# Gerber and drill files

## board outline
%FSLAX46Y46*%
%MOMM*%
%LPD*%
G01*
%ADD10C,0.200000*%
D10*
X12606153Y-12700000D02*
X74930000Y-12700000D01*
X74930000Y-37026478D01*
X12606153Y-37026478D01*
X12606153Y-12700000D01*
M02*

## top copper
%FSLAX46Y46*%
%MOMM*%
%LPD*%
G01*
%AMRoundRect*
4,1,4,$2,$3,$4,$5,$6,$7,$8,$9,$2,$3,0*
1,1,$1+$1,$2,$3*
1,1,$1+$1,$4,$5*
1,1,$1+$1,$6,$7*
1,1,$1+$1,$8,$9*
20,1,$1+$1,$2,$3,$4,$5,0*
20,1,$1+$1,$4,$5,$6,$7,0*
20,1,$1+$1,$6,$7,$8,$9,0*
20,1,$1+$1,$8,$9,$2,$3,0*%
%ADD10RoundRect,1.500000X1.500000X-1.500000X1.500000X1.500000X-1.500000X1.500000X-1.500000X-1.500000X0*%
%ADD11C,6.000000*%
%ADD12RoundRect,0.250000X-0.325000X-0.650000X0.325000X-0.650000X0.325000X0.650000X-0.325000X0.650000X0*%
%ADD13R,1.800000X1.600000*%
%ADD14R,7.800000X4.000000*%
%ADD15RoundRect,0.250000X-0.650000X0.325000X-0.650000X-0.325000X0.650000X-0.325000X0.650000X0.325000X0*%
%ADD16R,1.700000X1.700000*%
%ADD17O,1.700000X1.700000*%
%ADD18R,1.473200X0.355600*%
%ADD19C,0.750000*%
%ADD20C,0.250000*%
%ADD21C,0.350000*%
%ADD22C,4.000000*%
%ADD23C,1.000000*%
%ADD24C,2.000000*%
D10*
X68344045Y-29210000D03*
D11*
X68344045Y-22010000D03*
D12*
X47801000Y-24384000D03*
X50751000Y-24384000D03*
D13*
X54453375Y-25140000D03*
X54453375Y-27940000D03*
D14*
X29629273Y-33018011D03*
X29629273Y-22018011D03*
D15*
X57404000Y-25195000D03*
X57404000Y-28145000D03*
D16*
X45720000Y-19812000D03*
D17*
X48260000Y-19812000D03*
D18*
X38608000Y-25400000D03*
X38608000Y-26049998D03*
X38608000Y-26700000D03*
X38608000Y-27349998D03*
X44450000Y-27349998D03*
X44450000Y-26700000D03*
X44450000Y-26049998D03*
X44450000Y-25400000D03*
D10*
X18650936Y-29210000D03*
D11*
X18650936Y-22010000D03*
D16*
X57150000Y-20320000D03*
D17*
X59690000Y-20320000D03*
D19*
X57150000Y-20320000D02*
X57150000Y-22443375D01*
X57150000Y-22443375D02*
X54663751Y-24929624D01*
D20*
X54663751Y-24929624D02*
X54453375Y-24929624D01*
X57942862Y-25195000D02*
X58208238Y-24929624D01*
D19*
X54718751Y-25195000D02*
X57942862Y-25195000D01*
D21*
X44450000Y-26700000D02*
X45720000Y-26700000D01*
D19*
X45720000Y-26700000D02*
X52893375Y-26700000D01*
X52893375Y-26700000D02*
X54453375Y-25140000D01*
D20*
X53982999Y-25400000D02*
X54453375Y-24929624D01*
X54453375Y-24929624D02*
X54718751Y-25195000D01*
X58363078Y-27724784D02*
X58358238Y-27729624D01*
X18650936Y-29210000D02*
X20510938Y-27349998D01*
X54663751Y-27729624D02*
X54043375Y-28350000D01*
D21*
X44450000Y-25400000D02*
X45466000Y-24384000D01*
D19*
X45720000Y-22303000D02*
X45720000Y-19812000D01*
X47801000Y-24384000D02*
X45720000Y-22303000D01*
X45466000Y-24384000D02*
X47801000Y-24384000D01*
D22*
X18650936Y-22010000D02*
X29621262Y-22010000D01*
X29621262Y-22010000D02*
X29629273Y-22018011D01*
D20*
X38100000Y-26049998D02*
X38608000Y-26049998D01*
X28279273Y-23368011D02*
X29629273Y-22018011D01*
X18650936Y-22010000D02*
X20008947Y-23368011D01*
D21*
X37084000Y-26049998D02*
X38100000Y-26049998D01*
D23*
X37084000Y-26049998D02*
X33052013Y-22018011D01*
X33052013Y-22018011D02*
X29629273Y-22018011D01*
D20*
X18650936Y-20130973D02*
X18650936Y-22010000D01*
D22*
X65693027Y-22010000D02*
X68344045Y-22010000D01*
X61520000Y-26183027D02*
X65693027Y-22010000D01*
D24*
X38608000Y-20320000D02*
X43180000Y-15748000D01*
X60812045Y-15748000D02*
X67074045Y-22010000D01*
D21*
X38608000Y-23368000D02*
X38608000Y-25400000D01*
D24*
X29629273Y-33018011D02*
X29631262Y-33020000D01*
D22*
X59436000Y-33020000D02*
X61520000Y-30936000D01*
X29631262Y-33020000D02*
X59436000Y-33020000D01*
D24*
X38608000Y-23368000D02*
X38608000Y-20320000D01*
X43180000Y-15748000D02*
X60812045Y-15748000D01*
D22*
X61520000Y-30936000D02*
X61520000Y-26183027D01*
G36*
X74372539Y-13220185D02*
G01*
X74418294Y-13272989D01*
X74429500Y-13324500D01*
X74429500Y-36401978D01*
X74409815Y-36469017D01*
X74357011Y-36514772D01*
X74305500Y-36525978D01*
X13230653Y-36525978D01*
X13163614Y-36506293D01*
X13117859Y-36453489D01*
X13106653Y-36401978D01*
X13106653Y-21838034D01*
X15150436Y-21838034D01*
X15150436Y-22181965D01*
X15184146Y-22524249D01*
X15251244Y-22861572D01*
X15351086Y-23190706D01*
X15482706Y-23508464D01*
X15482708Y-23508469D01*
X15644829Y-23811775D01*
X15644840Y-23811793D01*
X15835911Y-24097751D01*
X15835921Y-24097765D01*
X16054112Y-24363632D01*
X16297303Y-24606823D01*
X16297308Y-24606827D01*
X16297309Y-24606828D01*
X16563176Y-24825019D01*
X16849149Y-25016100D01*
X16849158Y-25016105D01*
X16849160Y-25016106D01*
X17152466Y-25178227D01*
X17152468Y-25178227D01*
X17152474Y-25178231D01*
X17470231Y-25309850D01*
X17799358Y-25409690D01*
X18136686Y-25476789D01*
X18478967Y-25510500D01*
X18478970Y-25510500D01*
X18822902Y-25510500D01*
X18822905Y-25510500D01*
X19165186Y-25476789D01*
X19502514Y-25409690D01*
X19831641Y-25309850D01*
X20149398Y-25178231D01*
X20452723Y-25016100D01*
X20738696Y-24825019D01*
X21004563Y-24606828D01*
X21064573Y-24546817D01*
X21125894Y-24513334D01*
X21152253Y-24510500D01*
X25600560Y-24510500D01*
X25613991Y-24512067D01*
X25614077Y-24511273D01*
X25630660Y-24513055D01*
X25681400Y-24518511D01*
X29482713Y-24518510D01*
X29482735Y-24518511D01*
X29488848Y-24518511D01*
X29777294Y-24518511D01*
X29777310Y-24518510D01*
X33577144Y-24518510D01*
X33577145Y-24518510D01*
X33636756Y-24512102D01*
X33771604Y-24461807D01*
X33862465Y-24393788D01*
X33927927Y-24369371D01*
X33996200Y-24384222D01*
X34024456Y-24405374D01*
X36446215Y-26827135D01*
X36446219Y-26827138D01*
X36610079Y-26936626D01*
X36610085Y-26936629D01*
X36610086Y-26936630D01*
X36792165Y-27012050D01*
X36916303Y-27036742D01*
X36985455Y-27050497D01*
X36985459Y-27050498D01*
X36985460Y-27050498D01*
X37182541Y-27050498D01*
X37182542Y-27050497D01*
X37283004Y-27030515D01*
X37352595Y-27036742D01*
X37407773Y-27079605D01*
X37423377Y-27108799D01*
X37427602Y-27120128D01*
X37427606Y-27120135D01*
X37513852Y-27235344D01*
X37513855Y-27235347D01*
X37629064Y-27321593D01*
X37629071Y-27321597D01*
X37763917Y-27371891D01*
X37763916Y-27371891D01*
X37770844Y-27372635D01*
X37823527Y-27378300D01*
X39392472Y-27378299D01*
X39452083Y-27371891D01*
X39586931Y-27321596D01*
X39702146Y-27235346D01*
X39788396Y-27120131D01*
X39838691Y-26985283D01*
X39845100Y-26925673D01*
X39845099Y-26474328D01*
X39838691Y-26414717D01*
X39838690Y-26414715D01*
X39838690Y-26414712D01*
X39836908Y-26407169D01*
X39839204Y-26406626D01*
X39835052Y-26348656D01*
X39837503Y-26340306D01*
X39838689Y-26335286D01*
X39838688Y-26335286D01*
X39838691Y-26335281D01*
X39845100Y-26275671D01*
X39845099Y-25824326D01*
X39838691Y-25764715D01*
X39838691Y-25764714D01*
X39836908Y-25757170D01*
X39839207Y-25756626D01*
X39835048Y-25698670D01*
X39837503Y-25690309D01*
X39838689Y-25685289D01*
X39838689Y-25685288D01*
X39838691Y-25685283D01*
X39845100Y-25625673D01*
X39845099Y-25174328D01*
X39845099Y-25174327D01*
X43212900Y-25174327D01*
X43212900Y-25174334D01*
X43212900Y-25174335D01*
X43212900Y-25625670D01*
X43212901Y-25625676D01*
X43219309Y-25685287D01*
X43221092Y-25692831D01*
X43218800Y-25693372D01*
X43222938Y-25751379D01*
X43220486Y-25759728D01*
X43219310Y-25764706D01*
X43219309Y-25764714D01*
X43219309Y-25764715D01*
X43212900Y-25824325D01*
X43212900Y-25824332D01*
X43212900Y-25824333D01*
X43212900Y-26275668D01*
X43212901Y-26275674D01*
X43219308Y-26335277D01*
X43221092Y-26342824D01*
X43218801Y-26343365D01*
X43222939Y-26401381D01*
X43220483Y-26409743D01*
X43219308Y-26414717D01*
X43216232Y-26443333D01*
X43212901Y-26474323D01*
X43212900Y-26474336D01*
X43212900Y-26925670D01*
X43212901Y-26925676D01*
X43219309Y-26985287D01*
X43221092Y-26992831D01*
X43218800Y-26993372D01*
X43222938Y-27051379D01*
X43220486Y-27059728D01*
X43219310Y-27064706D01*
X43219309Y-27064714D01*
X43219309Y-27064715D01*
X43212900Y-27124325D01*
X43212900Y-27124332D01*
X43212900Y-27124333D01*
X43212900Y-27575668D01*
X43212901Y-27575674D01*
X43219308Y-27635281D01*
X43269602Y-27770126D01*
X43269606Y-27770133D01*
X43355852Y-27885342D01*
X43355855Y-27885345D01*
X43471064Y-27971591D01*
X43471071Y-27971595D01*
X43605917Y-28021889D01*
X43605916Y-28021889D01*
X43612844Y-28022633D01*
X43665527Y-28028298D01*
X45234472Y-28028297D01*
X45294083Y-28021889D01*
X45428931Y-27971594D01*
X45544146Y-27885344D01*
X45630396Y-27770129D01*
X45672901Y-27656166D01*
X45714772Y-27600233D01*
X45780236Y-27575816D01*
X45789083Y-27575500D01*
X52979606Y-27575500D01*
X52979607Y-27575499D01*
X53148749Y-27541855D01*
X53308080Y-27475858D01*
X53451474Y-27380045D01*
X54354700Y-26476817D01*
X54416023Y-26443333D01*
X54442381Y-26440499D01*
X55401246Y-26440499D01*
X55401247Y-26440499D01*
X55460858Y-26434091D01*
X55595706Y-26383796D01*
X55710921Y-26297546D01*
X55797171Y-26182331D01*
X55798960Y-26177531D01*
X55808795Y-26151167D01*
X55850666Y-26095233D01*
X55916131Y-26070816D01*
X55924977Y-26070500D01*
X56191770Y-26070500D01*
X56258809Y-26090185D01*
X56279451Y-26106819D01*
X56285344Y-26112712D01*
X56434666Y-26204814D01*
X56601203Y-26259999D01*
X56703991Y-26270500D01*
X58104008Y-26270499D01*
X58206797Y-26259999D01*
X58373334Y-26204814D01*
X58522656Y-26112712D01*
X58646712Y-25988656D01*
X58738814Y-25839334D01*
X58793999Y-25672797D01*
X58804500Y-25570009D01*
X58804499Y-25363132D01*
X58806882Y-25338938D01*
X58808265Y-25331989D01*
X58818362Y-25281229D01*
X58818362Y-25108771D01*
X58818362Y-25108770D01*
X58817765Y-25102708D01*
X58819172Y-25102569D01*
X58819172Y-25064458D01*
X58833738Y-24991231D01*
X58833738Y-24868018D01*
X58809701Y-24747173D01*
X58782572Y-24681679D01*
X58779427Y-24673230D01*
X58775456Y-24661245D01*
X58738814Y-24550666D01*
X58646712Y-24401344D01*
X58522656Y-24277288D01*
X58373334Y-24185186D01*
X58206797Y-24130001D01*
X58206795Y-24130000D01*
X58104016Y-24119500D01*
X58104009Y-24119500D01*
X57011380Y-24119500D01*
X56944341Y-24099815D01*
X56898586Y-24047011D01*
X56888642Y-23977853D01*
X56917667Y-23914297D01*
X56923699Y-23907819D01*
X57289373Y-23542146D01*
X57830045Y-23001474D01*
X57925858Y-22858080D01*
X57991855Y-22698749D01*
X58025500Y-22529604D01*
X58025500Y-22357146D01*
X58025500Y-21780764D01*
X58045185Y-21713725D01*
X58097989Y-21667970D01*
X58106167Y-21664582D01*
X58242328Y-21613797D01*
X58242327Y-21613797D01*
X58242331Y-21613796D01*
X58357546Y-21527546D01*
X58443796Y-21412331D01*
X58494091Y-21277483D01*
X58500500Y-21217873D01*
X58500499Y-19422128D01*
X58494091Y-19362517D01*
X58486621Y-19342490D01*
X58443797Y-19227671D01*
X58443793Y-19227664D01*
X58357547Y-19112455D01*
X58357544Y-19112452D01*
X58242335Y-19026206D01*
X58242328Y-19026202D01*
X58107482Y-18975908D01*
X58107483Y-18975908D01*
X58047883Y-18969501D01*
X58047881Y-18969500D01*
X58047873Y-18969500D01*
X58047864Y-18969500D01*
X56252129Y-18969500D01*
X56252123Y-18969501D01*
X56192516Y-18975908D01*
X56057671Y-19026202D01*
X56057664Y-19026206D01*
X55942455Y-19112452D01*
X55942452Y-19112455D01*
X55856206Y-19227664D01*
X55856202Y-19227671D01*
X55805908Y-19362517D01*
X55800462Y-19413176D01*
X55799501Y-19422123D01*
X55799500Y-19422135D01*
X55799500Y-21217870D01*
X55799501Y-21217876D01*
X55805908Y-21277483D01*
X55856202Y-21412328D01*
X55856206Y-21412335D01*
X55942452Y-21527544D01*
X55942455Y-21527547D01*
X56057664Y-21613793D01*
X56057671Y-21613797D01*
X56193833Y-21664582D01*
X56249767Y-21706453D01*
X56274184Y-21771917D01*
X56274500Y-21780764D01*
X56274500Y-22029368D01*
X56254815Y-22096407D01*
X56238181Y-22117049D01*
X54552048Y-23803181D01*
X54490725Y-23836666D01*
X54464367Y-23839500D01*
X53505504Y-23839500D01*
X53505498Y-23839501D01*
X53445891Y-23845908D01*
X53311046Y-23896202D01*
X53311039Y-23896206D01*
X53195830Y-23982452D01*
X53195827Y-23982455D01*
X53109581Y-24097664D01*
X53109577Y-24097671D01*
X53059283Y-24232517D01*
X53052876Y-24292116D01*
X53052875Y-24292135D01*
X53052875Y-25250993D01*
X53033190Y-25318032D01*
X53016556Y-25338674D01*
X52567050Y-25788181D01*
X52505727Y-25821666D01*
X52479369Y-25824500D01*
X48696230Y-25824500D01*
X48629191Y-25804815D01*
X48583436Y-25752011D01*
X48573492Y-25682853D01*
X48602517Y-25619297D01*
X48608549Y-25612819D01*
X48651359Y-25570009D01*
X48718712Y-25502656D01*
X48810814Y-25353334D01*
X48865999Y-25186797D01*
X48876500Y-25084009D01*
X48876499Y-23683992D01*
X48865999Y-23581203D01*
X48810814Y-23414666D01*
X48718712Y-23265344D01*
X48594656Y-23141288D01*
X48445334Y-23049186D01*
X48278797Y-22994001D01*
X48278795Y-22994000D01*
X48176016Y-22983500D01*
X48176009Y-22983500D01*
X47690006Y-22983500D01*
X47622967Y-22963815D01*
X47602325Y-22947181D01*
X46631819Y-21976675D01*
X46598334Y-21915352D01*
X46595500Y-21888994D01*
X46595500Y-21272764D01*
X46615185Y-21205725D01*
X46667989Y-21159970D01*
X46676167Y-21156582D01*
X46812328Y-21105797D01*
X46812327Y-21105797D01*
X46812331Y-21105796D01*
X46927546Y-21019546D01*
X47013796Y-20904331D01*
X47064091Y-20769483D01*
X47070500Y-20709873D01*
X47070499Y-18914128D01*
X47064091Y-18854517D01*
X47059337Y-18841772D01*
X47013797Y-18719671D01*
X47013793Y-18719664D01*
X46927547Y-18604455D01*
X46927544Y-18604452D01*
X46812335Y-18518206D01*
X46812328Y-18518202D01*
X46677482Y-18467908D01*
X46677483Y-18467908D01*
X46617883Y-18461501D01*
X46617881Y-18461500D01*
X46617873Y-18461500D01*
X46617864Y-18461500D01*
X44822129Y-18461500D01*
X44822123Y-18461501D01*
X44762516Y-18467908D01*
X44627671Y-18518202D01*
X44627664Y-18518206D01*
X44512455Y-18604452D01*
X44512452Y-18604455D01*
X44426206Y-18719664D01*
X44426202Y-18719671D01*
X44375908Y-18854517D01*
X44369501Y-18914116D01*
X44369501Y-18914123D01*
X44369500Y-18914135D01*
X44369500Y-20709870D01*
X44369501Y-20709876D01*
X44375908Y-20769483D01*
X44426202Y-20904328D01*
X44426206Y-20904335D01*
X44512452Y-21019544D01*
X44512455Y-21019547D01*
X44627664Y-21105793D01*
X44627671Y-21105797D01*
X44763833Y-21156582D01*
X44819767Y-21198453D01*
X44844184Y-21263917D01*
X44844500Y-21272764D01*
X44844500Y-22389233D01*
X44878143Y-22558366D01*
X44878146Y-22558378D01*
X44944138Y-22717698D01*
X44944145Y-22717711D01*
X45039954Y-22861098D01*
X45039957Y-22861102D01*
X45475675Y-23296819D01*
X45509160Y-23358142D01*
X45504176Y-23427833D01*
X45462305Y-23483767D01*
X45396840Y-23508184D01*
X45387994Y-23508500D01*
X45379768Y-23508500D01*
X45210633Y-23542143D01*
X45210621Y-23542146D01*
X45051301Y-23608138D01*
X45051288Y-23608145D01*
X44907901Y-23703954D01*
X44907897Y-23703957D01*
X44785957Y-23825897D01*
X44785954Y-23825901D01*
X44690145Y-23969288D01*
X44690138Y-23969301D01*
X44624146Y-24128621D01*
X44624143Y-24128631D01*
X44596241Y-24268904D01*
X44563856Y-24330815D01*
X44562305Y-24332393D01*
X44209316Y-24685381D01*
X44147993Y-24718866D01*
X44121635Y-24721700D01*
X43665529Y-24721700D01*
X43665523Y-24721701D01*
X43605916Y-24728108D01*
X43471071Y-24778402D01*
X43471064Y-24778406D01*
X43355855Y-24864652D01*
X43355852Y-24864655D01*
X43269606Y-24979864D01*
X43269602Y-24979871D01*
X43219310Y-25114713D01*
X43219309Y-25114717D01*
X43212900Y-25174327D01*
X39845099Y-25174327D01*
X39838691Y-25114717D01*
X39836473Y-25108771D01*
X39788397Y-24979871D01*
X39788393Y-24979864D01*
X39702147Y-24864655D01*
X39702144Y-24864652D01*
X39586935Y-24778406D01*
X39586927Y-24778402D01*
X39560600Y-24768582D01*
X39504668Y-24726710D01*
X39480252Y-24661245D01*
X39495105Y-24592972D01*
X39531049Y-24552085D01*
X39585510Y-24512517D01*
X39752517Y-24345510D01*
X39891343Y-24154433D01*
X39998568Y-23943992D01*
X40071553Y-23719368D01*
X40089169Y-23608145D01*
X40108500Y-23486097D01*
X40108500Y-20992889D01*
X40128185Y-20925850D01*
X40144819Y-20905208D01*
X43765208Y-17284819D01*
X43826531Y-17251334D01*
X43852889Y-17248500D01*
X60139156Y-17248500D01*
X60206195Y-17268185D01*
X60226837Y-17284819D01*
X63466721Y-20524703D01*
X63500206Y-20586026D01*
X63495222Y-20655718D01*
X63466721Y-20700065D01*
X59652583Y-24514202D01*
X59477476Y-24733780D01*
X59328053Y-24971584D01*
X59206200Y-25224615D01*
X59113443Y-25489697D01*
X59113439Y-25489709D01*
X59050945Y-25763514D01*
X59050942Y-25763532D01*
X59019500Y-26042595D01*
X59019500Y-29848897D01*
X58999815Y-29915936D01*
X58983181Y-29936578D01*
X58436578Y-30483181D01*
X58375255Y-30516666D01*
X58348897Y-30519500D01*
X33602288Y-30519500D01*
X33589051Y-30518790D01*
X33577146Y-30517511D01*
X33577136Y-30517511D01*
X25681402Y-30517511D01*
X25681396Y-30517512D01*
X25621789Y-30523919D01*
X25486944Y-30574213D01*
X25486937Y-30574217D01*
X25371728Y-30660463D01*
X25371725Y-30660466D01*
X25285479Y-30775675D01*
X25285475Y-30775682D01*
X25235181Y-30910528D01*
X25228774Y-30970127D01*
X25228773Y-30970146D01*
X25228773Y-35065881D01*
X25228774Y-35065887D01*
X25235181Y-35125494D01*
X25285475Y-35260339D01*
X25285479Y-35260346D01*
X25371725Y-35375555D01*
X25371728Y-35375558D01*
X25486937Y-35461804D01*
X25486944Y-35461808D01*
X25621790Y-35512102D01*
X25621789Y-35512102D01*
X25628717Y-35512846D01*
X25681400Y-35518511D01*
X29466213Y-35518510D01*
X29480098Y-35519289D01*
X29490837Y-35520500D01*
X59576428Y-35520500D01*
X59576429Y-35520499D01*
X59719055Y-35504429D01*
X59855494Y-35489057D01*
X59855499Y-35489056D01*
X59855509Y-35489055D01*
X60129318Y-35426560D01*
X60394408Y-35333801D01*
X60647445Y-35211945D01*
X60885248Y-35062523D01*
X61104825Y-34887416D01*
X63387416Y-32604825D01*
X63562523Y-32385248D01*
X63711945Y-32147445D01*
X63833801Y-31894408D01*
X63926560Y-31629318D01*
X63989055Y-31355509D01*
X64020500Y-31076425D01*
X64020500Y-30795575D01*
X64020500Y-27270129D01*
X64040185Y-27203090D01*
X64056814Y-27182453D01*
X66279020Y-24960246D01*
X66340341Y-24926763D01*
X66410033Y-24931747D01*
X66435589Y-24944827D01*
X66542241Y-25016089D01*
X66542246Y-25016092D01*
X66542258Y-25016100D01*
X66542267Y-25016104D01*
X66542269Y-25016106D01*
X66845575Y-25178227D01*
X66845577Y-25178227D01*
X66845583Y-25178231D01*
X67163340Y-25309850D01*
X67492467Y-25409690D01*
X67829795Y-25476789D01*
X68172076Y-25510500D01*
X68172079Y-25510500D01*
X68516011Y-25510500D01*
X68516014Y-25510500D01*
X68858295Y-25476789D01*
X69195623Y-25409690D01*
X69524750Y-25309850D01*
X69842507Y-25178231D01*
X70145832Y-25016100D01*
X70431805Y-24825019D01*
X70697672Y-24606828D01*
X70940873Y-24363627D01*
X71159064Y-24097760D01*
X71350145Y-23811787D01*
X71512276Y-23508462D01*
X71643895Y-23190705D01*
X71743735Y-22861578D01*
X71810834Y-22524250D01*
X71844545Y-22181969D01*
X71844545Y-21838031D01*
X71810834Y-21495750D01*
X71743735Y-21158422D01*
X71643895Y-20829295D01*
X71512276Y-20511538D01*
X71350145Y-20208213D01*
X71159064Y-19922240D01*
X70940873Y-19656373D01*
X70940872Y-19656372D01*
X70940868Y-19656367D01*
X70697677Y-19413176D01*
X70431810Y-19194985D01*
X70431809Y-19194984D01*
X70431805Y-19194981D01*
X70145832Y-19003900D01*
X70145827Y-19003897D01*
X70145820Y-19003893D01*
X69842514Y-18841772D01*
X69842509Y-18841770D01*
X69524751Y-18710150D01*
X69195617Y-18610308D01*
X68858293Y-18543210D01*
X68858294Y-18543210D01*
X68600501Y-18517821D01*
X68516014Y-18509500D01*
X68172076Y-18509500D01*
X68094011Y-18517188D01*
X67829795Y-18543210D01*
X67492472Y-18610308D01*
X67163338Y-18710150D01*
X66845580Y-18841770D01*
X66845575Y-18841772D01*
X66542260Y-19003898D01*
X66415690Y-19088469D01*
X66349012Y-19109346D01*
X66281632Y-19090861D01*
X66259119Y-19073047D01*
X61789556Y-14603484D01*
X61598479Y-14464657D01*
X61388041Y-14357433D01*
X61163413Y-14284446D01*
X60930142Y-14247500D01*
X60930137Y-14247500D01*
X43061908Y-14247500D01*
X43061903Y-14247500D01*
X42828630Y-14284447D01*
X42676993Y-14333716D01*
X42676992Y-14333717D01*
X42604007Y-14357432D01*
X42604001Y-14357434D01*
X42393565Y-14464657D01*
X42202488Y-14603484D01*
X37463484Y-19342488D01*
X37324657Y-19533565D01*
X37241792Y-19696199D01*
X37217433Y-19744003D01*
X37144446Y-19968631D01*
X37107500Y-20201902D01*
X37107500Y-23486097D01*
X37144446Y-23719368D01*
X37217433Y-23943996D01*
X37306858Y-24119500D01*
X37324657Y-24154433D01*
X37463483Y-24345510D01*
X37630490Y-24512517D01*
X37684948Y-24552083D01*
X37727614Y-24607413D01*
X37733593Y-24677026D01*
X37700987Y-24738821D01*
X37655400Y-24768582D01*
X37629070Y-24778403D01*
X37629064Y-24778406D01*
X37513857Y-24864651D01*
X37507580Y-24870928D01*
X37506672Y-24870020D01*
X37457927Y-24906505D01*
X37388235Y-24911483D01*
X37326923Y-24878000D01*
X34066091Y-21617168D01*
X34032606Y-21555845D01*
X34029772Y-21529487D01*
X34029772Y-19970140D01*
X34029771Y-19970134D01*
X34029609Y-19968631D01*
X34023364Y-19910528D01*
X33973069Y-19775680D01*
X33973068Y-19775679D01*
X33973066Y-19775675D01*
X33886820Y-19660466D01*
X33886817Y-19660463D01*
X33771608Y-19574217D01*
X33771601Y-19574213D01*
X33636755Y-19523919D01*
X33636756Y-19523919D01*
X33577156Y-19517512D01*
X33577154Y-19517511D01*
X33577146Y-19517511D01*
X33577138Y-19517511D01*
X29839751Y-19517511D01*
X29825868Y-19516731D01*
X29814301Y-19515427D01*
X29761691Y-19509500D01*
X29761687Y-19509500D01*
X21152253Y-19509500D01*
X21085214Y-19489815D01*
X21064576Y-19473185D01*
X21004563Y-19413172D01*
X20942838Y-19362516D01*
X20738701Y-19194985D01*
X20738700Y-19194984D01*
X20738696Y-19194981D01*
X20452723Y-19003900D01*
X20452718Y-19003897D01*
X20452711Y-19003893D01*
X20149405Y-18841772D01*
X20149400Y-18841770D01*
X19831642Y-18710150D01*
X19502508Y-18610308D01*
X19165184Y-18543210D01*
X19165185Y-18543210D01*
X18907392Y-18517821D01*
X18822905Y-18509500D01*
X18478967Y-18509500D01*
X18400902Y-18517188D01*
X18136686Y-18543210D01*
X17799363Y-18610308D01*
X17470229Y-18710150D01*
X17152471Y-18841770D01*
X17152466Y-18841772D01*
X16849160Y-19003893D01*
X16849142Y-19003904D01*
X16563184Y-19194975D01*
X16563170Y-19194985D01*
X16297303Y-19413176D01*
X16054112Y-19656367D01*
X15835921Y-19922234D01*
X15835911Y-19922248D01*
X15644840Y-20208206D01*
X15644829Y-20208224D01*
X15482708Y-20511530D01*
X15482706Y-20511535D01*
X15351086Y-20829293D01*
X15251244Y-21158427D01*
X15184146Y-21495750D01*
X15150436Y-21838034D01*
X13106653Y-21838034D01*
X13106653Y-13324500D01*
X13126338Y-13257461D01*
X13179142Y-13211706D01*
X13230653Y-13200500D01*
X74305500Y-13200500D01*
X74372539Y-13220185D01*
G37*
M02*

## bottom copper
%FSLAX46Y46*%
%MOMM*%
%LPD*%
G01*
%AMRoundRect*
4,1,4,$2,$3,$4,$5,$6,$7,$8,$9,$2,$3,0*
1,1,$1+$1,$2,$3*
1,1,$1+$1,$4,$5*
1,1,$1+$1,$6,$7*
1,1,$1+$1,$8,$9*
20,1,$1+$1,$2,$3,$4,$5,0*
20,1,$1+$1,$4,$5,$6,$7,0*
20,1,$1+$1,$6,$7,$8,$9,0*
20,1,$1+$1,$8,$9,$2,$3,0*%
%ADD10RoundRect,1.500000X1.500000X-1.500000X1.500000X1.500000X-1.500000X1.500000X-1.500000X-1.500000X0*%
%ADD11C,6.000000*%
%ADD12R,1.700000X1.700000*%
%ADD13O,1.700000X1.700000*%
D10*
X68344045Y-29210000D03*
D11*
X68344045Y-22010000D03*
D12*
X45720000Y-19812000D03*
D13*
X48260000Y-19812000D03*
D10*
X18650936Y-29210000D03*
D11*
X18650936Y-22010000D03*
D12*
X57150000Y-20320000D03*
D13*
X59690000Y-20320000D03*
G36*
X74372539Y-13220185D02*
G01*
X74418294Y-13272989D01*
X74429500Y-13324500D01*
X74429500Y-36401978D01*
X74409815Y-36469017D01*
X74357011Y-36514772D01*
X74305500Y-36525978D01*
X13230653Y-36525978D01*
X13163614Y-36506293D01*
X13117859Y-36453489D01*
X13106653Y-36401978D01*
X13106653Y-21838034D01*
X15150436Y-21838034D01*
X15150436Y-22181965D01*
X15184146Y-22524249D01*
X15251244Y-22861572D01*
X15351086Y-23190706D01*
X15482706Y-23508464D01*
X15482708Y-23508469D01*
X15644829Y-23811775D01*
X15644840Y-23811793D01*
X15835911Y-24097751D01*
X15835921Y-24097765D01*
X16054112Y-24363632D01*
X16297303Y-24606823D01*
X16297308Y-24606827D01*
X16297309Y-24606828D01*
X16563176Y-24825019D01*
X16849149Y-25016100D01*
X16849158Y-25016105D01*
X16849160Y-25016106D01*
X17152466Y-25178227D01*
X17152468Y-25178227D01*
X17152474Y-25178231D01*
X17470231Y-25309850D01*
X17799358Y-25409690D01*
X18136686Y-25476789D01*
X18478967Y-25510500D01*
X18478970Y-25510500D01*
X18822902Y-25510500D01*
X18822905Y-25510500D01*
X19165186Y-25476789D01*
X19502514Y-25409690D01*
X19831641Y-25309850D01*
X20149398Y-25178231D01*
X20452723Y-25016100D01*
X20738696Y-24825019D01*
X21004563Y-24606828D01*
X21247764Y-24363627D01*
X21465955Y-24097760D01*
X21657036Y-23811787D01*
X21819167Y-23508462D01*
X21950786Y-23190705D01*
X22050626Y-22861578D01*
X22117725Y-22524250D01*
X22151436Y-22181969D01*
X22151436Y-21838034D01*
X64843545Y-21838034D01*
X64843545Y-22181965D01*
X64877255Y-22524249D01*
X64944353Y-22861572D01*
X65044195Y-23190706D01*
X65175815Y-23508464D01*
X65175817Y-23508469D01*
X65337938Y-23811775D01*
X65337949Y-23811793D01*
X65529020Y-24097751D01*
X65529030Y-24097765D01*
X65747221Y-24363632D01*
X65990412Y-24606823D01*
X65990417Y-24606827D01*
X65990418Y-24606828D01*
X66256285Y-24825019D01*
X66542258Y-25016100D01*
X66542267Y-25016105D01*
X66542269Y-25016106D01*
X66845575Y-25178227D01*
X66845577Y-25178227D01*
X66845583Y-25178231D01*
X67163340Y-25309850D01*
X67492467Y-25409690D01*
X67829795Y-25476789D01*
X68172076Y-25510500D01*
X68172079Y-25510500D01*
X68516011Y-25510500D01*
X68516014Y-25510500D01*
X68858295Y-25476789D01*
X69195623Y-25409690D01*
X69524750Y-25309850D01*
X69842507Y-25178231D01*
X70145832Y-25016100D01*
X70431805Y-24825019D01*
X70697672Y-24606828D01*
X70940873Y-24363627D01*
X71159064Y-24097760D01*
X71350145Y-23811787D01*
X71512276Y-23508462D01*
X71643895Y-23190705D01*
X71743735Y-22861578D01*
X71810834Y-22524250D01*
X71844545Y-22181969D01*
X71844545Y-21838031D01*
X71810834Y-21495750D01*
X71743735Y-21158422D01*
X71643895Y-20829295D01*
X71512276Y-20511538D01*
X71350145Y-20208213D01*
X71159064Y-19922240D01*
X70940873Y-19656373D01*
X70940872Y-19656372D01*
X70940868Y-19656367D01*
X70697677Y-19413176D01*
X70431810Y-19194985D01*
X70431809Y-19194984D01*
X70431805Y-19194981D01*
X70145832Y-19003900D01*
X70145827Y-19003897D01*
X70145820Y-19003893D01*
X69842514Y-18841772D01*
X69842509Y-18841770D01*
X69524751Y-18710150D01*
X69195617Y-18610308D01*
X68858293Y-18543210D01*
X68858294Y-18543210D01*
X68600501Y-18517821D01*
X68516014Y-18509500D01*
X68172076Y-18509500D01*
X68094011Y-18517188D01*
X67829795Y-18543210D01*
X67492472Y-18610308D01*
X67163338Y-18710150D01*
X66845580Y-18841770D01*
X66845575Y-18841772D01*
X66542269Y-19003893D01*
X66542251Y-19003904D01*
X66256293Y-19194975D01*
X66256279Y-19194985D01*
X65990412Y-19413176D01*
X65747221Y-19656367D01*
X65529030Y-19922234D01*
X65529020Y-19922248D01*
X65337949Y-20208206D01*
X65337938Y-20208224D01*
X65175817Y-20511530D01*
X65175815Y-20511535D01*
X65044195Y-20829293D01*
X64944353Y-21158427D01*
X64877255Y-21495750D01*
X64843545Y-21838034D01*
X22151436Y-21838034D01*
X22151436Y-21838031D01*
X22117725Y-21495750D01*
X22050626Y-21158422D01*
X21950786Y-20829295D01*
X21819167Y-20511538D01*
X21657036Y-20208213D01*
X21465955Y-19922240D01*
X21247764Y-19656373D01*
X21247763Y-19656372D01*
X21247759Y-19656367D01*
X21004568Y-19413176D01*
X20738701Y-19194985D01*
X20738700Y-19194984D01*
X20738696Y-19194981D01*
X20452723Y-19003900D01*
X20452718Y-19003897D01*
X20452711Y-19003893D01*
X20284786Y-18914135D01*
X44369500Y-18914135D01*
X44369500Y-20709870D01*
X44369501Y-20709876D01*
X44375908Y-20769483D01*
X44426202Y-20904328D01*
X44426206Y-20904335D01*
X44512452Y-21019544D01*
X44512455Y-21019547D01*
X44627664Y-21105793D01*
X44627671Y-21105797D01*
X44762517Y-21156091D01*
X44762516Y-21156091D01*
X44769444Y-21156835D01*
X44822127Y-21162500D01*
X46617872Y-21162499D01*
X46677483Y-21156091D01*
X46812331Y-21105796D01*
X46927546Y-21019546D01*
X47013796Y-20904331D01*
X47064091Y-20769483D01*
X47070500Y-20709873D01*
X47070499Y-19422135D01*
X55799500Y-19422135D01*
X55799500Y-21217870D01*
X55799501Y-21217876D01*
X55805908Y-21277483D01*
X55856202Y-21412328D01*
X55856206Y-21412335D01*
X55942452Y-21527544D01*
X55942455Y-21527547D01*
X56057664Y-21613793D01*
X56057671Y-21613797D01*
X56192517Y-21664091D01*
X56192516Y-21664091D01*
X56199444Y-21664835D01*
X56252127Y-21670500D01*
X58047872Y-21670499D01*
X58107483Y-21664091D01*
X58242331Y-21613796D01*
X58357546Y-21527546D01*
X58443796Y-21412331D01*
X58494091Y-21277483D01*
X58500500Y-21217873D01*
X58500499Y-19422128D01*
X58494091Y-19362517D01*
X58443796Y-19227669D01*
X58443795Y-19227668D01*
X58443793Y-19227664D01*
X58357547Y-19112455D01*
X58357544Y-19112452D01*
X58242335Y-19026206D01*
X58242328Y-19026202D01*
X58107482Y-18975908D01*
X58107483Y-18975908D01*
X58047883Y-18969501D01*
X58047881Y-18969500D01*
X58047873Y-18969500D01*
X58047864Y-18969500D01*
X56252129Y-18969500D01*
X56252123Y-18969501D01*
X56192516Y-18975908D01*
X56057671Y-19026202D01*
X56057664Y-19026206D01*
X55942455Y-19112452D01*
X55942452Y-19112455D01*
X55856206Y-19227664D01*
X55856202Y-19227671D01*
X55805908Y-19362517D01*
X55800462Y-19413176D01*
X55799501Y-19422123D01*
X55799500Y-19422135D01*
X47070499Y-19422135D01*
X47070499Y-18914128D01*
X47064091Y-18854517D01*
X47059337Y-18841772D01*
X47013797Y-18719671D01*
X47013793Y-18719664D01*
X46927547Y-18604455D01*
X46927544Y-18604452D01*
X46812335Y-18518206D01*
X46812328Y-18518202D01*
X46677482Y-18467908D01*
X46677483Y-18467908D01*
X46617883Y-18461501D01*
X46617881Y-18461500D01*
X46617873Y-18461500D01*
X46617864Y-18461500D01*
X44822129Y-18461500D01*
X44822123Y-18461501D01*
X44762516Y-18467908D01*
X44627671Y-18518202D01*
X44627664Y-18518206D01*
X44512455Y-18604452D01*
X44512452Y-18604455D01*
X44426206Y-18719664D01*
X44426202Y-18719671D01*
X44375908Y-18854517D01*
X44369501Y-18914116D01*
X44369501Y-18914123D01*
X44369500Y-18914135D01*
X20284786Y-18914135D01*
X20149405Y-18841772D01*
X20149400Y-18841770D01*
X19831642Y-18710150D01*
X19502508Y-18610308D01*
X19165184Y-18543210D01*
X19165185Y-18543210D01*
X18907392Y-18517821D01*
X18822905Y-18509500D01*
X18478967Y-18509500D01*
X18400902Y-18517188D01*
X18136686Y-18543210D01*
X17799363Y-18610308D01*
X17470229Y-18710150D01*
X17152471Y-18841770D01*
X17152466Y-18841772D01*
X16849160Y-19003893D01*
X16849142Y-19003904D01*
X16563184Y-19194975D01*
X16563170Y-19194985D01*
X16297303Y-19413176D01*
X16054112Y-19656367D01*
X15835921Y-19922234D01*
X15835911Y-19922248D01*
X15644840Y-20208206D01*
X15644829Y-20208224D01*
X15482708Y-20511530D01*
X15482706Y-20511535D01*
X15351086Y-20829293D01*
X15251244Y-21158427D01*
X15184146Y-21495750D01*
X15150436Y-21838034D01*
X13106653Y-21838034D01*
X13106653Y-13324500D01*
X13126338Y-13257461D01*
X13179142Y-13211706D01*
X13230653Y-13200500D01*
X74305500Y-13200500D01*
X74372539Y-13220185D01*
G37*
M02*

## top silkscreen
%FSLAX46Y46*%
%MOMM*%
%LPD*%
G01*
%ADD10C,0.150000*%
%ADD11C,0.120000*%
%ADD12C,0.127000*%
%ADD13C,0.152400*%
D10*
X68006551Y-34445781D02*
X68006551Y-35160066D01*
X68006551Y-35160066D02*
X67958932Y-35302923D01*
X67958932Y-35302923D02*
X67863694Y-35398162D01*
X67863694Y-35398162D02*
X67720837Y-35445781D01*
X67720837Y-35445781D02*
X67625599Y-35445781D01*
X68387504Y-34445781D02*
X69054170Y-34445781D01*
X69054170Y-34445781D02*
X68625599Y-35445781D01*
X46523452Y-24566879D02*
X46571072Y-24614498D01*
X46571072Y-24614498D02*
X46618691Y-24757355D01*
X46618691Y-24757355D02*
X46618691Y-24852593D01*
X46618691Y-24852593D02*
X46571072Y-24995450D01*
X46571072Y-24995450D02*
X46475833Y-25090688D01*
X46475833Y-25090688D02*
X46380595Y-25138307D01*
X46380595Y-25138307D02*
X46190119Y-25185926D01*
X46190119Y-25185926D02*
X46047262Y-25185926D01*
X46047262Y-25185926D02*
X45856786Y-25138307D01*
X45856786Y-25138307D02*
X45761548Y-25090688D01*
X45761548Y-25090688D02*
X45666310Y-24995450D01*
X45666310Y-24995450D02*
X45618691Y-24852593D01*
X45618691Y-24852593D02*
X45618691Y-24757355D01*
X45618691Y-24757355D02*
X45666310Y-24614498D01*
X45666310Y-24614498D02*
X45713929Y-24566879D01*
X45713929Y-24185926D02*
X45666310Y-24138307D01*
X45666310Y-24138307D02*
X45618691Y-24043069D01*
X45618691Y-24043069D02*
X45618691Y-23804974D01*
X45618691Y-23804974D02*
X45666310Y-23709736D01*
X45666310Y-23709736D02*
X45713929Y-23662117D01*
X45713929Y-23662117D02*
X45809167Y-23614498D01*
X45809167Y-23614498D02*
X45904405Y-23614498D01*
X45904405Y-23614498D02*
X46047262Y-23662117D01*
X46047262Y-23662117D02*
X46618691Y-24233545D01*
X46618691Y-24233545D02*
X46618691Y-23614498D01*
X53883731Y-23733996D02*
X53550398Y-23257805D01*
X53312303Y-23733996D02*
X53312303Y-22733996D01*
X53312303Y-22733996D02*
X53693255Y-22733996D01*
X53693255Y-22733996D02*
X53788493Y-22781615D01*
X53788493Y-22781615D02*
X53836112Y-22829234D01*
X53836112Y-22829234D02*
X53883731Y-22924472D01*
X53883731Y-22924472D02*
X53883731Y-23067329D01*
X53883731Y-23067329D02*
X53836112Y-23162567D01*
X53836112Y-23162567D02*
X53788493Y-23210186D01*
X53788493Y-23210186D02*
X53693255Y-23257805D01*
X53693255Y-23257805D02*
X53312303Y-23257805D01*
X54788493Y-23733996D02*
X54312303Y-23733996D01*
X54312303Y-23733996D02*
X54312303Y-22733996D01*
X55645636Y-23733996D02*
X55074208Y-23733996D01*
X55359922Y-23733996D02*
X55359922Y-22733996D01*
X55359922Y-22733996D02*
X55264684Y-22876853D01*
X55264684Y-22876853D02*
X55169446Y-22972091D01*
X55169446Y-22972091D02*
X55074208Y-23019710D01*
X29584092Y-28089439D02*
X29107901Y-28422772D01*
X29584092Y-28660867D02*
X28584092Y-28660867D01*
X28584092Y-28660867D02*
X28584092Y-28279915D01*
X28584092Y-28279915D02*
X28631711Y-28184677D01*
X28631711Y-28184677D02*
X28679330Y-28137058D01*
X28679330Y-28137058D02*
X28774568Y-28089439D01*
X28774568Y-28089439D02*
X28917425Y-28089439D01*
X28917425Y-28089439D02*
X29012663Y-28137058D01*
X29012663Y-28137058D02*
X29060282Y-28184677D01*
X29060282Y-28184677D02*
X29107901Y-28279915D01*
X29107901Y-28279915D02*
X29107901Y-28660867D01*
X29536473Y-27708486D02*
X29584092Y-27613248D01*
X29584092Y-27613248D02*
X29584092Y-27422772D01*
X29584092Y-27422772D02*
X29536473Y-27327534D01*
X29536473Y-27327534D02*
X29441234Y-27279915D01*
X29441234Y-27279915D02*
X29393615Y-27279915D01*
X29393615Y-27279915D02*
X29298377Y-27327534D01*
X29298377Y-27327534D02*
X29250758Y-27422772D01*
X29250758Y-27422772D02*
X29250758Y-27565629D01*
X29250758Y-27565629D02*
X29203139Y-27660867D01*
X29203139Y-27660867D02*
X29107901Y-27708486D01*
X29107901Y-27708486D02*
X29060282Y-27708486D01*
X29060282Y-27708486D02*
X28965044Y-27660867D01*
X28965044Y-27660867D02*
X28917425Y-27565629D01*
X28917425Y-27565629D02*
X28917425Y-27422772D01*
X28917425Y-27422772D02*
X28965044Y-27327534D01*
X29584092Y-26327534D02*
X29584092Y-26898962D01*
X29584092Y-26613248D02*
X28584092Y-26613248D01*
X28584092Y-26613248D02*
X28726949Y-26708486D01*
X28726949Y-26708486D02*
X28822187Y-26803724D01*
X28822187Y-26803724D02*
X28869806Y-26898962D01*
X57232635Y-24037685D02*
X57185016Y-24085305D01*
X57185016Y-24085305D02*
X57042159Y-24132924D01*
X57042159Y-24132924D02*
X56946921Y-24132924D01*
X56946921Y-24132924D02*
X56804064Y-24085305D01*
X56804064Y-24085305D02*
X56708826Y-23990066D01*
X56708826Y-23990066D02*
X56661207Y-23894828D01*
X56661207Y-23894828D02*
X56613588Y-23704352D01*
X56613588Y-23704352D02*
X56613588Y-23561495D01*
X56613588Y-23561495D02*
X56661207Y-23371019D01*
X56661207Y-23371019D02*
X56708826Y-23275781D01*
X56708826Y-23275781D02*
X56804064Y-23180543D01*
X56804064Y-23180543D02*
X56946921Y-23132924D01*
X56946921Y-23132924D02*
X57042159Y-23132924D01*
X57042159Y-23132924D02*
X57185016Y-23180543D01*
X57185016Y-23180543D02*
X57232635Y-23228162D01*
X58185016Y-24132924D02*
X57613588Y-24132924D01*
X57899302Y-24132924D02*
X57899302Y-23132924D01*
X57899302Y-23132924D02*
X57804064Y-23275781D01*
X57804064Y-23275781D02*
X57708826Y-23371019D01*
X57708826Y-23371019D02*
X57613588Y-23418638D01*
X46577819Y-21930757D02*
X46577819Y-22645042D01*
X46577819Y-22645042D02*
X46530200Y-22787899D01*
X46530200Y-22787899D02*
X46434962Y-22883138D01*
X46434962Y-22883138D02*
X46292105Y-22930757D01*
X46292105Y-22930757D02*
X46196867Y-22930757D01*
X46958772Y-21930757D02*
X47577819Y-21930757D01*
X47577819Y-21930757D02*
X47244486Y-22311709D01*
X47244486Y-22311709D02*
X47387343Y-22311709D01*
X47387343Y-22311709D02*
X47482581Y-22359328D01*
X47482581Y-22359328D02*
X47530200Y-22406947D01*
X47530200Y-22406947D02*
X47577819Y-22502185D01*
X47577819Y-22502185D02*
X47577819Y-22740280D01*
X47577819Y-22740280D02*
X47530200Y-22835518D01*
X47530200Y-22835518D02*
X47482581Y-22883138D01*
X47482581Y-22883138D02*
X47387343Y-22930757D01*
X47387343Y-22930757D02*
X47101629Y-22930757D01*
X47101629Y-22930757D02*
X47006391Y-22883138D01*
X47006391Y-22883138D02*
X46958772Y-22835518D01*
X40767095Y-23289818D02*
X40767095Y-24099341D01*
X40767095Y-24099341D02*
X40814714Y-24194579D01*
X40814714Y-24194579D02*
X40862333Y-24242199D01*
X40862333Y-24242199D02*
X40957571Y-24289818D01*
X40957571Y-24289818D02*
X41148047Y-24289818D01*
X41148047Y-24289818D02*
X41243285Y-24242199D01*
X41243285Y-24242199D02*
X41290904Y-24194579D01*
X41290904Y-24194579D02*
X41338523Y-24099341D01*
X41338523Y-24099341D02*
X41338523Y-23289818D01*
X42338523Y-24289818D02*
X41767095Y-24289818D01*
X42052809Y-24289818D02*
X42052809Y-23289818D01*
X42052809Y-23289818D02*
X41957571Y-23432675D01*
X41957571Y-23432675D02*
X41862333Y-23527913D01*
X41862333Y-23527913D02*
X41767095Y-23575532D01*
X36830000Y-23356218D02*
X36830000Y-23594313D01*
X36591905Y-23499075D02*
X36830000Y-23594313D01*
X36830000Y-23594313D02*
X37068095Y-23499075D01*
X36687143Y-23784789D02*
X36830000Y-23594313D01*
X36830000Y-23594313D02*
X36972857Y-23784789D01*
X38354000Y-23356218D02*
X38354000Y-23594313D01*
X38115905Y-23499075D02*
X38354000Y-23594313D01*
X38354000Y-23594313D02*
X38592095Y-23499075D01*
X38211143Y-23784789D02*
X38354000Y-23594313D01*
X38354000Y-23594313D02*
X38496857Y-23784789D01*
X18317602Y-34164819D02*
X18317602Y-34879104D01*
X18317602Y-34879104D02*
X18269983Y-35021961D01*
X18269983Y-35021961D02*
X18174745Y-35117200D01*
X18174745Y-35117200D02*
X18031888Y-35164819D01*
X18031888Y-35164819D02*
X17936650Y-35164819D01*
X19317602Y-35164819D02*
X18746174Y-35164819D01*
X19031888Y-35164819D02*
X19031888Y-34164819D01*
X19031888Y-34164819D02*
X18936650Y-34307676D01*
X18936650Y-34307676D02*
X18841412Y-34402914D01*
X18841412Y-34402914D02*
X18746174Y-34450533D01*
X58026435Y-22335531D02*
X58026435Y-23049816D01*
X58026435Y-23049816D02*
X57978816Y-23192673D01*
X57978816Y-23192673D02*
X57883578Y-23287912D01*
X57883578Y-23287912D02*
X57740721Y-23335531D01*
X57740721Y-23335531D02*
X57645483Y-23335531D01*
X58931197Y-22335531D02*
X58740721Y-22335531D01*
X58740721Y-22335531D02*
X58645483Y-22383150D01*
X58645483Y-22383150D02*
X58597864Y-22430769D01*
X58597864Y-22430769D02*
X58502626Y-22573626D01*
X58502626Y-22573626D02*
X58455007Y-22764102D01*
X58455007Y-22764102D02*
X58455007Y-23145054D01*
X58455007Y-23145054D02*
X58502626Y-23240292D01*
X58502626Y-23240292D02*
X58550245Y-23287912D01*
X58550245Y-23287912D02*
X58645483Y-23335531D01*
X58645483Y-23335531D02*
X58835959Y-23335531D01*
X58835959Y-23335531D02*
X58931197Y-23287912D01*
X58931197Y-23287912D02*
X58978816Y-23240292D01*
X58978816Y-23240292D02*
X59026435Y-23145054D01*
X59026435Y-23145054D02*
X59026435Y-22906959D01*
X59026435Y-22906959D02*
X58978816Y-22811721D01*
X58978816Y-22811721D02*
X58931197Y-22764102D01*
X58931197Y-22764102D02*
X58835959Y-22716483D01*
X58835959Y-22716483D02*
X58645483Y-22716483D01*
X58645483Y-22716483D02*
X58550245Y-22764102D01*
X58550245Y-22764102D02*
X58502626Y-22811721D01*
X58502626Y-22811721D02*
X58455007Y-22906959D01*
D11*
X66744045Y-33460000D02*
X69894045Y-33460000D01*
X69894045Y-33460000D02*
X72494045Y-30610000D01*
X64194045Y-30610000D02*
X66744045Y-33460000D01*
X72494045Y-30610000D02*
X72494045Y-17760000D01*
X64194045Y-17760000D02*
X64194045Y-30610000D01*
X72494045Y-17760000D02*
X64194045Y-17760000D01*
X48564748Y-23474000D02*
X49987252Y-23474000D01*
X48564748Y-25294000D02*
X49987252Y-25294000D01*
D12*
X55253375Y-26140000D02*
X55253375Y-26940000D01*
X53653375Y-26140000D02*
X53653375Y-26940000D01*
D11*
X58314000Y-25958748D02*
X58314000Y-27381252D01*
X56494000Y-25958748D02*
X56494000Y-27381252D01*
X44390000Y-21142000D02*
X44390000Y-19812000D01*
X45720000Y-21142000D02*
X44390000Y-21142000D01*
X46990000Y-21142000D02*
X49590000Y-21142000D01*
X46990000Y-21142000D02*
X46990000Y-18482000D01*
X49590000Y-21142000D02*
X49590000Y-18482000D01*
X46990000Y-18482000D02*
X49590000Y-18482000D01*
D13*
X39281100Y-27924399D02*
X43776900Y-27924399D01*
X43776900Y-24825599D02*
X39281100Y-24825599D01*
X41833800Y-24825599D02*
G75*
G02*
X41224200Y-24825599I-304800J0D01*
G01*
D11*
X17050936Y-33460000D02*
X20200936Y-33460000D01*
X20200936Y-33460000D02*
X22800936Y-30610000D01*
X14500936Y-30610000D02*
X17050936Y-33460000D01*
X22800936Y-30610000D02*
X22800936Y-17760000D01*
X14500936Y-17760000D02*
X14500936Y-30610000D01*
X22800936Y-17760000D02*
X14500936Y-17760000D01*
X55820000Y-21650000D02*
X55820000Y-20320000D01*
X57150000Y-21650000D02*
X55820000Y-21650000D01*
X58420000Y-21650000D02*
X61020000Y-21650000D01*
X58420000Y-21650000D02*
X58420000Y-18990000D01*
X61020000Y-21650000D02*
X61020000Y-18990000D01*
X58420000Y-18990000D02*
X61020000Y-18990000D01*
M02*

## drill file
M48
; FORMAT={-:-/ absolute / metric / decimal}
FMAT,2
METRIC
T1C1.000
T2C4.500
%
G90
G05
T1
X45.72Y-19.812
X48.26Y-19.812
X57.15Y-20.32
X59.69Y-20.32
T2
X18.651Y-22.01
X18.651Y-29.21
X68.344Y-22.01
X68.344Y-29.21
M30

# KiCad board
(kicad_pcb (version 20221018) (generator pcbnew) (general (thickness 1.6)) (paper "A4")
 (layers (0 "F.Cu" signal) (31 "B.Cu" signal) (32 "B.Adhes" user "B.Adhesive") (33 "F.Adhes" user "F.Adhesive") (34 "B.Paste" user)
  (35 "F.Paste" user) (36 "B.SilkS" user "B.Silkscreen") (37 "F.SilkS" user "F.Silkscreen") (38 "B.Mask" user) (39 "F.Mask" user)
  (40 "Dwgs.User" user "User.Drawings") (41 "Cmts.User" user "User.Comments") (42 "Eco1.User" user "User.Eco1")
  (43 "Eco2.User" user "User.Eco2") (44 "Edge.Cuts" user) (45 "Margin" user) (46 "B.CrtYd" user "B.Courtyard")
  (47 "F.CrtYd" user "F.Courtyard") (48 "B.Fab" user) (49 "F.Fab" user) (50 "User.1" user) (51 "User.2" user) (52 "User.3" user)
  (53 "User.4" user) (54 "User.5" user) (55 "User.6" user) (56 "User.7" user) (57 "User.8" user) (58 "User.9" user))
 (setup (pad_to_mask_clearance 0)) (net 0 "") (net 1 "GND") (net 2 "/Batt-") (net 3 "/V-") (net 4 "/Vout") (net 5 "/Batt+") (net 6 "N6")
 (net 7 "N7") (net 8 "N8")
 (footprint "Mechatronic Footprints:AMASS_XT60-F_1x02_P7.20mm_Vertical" (layer "F.Cu") (at 68.344045 29.21 90)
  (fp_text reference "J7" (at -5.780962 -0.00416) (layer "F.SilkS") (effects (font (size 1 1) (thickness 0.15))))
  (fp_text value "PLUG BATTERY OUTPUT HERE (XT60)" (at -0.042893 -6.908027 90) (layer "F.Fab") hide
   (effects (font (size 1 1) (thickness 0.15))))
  (fp_line (start -4.25 -1.6) (end -4.25 1.55) (stroke (width 0.12) (type solid)) (layer "F.SilkS"))
  (fp_line (start -4.25 1.55) (end -1.4 4.15) (stroke (width 0.12) (type solid)) (layer "F.SilkS"))
  (fp_line (start -1.4 -4.15) (end -4.25 -1.6) (stroke (width 0.12) (type solid)) (layer "F.SilkS"))
  (fp_line (start -1.4 4.15) (end 11.45 4.15) (stroke (width 0.12) (type solid)) (layer "F.SilkS"))
  (fp_line (start 11.45 -4.15) (end -1.4 -4.15) (stroke (width 0.12) (type solid)) (layer "F.SilkS"))
  (fp_line (start 11.45 4.15) (end 11.45 -4.15) (stroke (width 0.12) (type solid)) (layer "F.SilkS"))
  (pad "1" thru_hole roundrect (at 0 0 90) (size 6 6) (drill 4.5) (layers "*.Cu" "*.Mask") (roundrect_rratio 0.25) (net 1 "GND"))
  (pad "2" thru_hole circle (at 7.2 0 90) (size 6 6) (drill 4.5) (layers "*.Cu" "*.Mask") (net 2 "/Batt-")))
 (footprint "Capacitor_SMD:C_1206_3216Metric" (layer "F.Cu") (at 49.276 24.384)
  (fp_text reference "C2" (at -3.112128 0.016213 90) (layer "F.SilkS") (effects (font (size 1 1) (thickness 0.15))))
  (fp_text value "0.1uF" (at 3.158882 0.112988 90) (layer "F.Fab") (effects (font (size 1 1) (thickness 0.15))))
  (fp_line (start -0.711252 -0.91) (end 0.711252 -0.91) (stroke (width 0.12) (type solid)) (layer "F.SilkS"))
  (fp_line (start -0.711252 0.91) (end 0.711252 0.91) (stroke (width 0.12) (type solid)) (layer "F.SilkS"))
  (pad "1" smd roundrect (at -1.475 0) (size 1.15 1.8) (layers "F.Cu" "F.Paste" "F.Mask") (roundrect_rratio 0.2173913043) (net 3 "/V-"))
  (pad "2" smd roundrect (at 1.475 0) (size 1.15 1.8) (layers "F.Cu" "F.Paste" "F.Mask") (roundrect_rratio 0.2173913043) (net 1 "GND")))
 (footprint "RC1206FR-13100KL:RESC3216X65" (layer "F.Cu") (at 54.453375 26.54 -90)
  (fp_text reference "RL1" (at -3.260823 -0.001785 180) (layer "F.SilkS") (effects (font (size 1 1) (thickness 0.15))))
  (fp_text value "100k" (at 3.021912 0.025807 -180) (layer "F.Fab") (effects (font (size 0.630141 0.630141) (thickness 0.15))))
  (fp_line (start -0.4 -0.8) (end 0.4 -0.8) (stroke (width 0.127) (type solid)) (layer "F.SilkS"))
  (fp_line (start -0.4 0.8) (end 0.4 0.8) (stroke (width 0.127) (type solid)) (layer "F.SilkS"))
  (pad "1" smd rect (at -1.4 0 270) (size 1.6 1.8) (layers "F.Cu" "F.Paste" "F.Mask") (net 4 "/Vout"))
  (pad "2" smd rect (at 1.4 0 270) (size 1.6 1.8) (layers "F.Cu" "F.Paste" "F.Mask") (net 1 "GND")))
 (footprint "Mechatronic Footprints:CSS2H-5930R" (layer "F.Cu") (at 29.629273 27.518011 90)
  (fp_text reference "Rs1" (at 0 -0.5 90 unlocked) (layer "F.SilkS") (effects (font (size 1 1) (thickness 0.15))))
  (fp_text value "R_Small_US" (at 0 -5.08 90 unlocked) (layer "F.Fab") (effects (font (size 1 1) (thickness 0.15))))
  (pad "1" smd rect (at -5.5 0 180) (size 7.8 4) (layers "F.Cu" "F.Paste" "F.Mask") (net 2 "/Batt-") (thermal_bridge_angle 45))
  (pad "2" smd rect (at 5.5 0 180) (size 7.8 4) (layers "F.Cu" "F.Paste" "F.Mask") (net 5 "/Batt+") (thermal_bridge_angle 45)))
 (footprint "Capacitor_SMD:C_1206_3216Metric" (layer "F.Cu") (at 57.404 26.67 -90)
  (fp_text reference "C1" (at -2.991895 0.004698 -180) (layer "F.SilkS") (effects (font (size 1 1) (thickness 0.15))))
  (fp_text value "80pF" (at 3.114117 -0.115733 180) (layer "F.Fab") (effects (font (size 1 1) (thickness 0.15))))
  (fp_line (start -0.711252 -0.91) (end 0.711252 -0.91) (stroke (width 0.12) (type solid)) (layer "F.SilkS"))
  (fp_line (start -0.711252 0.91) (end 0.711252 0.91) (stroke (width 0.12) (type solid)) (layer "F.SilkS"))
  (pad "1" smd roundrect (at -1.475 0 270) (size 1.15 1.8) (layers "F.Cu" "F.Paste" "F.Mask") (roundrect_rratio 0.2173913043)
   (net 4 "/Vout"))
  (pad "2" smd roundrect (at 1.475 0 270) (size 1.15 1.8) (layers "F.Cu" "F.Paste" "F.Mask") (roundrect_rratio 0.2173913043) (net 1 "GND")))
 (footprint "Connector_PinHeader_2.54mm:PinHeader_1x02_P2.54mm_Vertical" (layer "F.Cu") (at 45.72 19.812 90)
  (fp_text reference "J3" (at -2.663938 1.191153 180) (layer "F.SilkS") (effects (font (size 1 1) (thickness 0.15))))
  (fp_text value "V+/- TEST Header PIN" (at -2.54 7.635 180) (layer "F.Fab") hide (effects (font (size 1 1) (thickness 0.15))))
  (fp_line (start -1.33 -1.33) (end 0 -1.33) (stroke (width 0.12) (type solid)) (layer "F.SilkS"))
  (fp_line (start -1.33 0) (end -1.33 -1.33) (stroke (width 0.12) (type solid)) (layer "F.SilkS"))
  (fp_line (start -1.33 1.27) (end -1.33 3.87) (stroke (width 0.12) (type solid)) (layer "F.SilkS"))
  (fp_line (start -1.33 1.27) (end 1.33 1.27) (stroke (width 0.12) (type solid)) (layer "F.SilkS"))
  (fp_line (start -1.33 3.87) (end 1.33 3.87) (stroke (width 0.12) (type solid)) (layer "F.SilkS"))
  (fp_line (start 1.33 1.27) (end 1.33 3.87) (stroke (width 0.12) (type solid)) (layer "F.SilkS"))
  (pad "1" thru_hole rect (at 0 0 90) (size 1.7 1.7) (drill 1) (layers "*.Cu" "*.Mask") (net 3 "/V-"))
  (pad "2" thru_hole oval (at 0 2.54 90) (size 1.7 1.7) (drill 1) (layers "*.Cu" "*.Mask") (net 1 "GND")))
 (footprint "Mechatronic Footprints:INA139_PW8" (layer "F.Cu") (at 41.529 26.374999)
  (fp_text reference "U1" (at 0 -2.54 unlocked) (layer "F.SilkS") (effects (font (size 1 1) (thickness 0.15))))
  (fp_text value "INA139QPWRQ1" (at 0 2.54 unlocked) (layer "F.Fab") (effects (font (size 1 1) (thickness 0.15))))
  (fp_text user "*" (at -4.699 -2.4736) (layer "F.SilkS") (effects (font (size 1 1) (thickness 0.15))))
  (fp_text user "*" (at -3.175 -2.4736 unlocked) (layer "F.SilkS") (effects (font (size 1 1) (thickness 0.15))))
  (fp_line (start -2.2479 1.5494) (end 2.2479 1.5494) (stroke (width 0.1524) (type solid)) (layer "F.SilkS"))
  (fp_line (start 2.2479 -1.5494) (end -2.2479 -1.5494) (stroke (width 0.1524) (type solid)) (layer "F.SilkS"))
  (fp_arc (start 0.3048 -1.5494) (mid 0 -1.2446) (end -0.3048 -1.5494) (stroke (width 0.1524) (type solid)) (layer "F.SilkS"))
  (pad "1" smd rect (at -2.921 -0.974999) (size 1.4732 0.3556) (layers "F.Cu" "F.Paste" "F.Mask") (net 2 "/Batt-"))
  (pad "2" smd rect (at -2.921 -0.325001) (size 1.4732 0.3556) (layers "F.Cu" "F.Paste" "F.Mask") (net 5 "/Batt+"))
  (pad "3" smd rect (at -2.921 0.325001) (size 1.4732 0.3556) (layers "F.Cu" "F.Paste" "F.Mask") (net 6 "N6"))
  (pad "4" smd rect (at -2.921 0.974999) (size 1.4732 0.3556) (layers "F.Cu" "F.Paste" "F.Mask") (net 1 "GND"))
  (pad "5" smd rect (at 2.921 0.974999) (size 1.4732 0.3556) (layers "F.Cu" "F.Paste" "F.Mask") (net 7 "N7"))
  (pad "6" smd rect (at 2.921 0.325001) (size 1.4732 0.3556) (layers "F.Cu" "F.Paste" "F.Mask") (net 4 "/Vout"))
  (pad "7" smd rect (at 2.921 -0.325001) (size 1.4732 0.3556) (layers "F.Cu" "F.Paste" "F.Mask") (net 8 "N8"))
  (pad "8" smd rect (at 2.921 -0.974999) (size 1.4732 0.3556) (layers "F.Cu" "F.Paste" "F.Mask") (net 3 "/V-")))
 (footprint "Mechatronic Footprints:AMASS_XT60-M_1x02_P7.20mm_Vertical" (layer "F.Cu") (at 18.650936 29.21 90)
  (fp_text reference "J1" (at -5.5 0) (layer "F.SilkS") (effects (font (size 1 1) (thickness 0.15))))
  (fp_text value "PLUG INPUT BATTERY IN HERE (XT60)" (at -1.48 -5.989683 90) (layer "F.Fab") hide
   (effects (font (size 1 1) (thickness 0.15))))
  (fp_line (start -4.25 -1.6) (end -4.25 1.55) (stroke (width 0.12) (type solid)) (layer "F.SilkS"))
  (fp_line (start -4.25 1.55) (end -1.4 4.15) (stroke (width 0.12) (type solid)) (layer "F.SilkS"))
  (fp_line (start -1.4 -4.15) (end -4.25 -1.6) (stroke (width 0.12) (type solid)) (layer "F.SilkS"))
  (fp_line (start -1.4 4.15) (end 11.45 4.15) (stroke (width 0.12) (type solid)) (layer "F.SilkS"))
  (fp_line (start 11.45 -4.15) (end -1.4 -4.15) (stroke (width 0.12) (type solid)) (layer "F.SilkS"))
  (fp_line (start 11.45 4.15) (end 11.45 -4.15) (stroke (width 0.12) (type solid)) (layer "F.SilkS"))
  (pad "1" thru_hole roundrect (at 0 0 90) (size 6 6) (drill 4.5) (layers "*.Cu" "*.Mask") (roundrect_rratio 0.25) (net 1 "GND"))
  (pad "2" thru_hole circle (at 7.2 0 90) (size 6 6) (drill 4.5) (layers "*.Cu" "*.Mask") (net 5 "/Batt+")))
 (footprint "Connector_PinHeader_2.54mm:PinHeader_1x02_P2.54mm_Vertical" (layer "F.Cu") (at 57.15 20.32 90)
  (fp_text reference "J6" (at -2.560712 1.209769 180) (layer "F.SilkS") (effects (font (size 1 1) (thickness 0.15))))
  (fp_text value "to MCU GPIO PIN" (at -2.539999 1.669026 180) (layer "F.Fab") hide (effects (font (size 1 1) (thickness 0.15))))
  (fp_line (start -1.33 -1.33) (end 0 -1.33) (stroke (width 0.12) (type solid)) (layer "F.SilkS"))
  (fp_line (start -1.33 0) (end -1.33 -1.33) (stroke (width 0.12) (type solid)) (layer "F.SilkS"))
  (fp_line (start -1.33 1.27) (end -1.33 3.87) (stroke (width 0.12) (type solid)) (layer "F.SilkS"))
  (fp_line (start -1.33 1.27) (end 1.33 1.27) (stroke (width 0.12) (type solid)) (layer "F.SilkS"))
  (fp_line (start -1.33 3.87) (end 1.33 3.87) (stroke (width 0.12) (type solid)) (layer "F.SilkS"))
  (fp_line (start 1.33 1.27) (end 1.33 3.87) (stroke (width 0.12) (type solid)) (layer "F.SilkS"))
  (pad "1" thru_hole rect (at 0 0 90) (size 1.7 1.7) (drill 1) (layers "*.Cu" "*.Mask") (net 4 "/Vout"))
  (pad "2" thru_hole oval (at 0 2.54 90) (size 1.7 1.7) (drill 1) (layers "*.Cu" "*.Mask") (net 1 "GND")))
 (gr_rect (start 12.606153 12.7) (end 74.93 37.026478) (stroke (width 0.2) (type default)) (fill none) (layer "Edge.Cuts"))
 (segment (start 57.15 20.32) (end 57.15 22.443375) (width 0.75) (layer "F.Cu") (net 4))
 (segment (start 57.15 22.443375) (end 54.663751 24.929624) (width 0.75) (layer "F.Cu") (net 4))
 (segment (start 54.663751 24.929624) (end 54.453375 24.929624) (width 0.25) (layer "F.Cu") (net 4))
 (segment (start 57.942862 25.195) (end 58.208238 24.929624) (width 0.25) (layer "F.Cu") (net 4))
 (segment (start 54.718751 25.195) (end 57.942862 25.195) (width 0.75) (layer "F.Cu") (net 4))
 (segment (start 44.45 26.7) (end 45.72 26.7) (width 0.35) (layer "F.Cu") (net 4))
 (segment (start 45.72 26.7) (end 52.893375 26.7) (width 0.75) (layer "F.Cu") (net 4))
 (segment (start 52.893375 26.7) (end 54.453375 25.14) (width 0.75) (layer "F.Cu") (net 4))
 (segment (start 53.982999 25.4) (end 54.453375 24.929624) (width 0.25) (layer "F.Cu") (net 4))
 (segment (start 54.453375 24.929624) (end 54.718751 25.195) (width 0.25) (layer "F.Cu") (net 4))
 (segment (start 58.363078 27.724784) (end 58.358238 27.729624) (width 0.25) (layer "F.Cu") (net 1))
 (segment (start 18.650936 29.21) (end 20.510938 27.349998) (width 0.25) (layer "F.Cu") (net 1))
 (segment (start 54.663751 27.729624) (end 54.043375 28.35) (width 0.25) (layer "F.Cu") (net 1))
 (segment (start 44.45 25.4) (end 45.466 24.384) (width 0.35) (layer "F.Cu") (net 3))
 (segment (start 45.72 22.303) (end 45.72 19.812) (width 0.75) (layer "F.Cu") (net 3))
 (segment (start 47.801 24.384) (end 45.72 22.303) (width 0.75) (layer "F.Cu") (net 3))
 (segment (start 45.466 24.384) (end 47.801 24.384) (width 0.75) (layer "F.Cu") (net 3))
 (segment (start 18.650936 22.01) (end 29.621262 22.01) (width 4) (layer "F.Cu") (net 5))
 (segment (start 29.621262 22.01) (end 29.629273 22.018011) (width 4) (layer "F.Cu") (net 5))
 (segment (start 38.1 26.049998) (end 38.608 26.049998) (width 0.25) (layer "F.Cu") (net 5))
 (segment (start 28.279273 23.368011) (end 29.629273 22.018011) (width 0.25) (layer "F.Cu") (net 5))
 (segment (start 18.650936 22.01) (end 20.008947 23.368011) (width 0.25) (layer "F.Cu") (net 5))
 (segment (start 37.084 26.049998) (end 38.1 26.049998) (width 0.35) (layer "F.Cu") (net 5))
 (segment (start 37.084 26.049998) (end 33.052013 22.018011) (width 1) (layer "F.Cu") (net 5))
 (segment (start 33.052013 22.018011) (end 29.629273 22.018011) (width 1) (layer "F.Cu") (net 5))
 (segment (start 18.650936 20.130973) (end 18.650936 22.01) (width 0.25) (layer "F.Cu") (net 5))
 (segment (start 65.693027 22.01) (end 68.344045 22.01) (width 4) (layer "F.Cu") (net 2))
 (segment (start 61.52 26.183027) (end 65.693027 22.01) (width 4) (layer "F.Cu") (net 2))
 (segment (start 38.608 20.32) (end 43.18 15.748) (width 2) (layer "F.Cu") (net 2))
 (segment (start 60.812045 15.748) (end 67.074045 22.01) (width 2) (layer "F.Cu") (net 2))
 (segment (start 38.608 23.368) (end 38.608 25.4) (width 0.35) (layer "F.Cu") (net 2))
 (segment (start 29.629273 33.018011) (end 29.631262 33.02) (width 2) (layer "F.Cu") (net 2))
 (segment (start 59.436 33.02) (end 61.52 30.936) (width 4) (layer "F.Cu") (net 2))
 (segment (start 29.631262 33.02) (end 59.436 33.02) (width 4) (layer "F.Cu") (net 2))
 (segment (start 38.608 23.368) (end 38.608 20.32) (width 2) (layer "F.Cu") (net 2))
 (segment (start 43.18 15.748) (end 60.812045 15.748) (width 2) (layer "F.Cu") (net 2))
 (segment (start 61.52 30.936) (end 61.52 26.183027) (width 4) (layer "F.Cu") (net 2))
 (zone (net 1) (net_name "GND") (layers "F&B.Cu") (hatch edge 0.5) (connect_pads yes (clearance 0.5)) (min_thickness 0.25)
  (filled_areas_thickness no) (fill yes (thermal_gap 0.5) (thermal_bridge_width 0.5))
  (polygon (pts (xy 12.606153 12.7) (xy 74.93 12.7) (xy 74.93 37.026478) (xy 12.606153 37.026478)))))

